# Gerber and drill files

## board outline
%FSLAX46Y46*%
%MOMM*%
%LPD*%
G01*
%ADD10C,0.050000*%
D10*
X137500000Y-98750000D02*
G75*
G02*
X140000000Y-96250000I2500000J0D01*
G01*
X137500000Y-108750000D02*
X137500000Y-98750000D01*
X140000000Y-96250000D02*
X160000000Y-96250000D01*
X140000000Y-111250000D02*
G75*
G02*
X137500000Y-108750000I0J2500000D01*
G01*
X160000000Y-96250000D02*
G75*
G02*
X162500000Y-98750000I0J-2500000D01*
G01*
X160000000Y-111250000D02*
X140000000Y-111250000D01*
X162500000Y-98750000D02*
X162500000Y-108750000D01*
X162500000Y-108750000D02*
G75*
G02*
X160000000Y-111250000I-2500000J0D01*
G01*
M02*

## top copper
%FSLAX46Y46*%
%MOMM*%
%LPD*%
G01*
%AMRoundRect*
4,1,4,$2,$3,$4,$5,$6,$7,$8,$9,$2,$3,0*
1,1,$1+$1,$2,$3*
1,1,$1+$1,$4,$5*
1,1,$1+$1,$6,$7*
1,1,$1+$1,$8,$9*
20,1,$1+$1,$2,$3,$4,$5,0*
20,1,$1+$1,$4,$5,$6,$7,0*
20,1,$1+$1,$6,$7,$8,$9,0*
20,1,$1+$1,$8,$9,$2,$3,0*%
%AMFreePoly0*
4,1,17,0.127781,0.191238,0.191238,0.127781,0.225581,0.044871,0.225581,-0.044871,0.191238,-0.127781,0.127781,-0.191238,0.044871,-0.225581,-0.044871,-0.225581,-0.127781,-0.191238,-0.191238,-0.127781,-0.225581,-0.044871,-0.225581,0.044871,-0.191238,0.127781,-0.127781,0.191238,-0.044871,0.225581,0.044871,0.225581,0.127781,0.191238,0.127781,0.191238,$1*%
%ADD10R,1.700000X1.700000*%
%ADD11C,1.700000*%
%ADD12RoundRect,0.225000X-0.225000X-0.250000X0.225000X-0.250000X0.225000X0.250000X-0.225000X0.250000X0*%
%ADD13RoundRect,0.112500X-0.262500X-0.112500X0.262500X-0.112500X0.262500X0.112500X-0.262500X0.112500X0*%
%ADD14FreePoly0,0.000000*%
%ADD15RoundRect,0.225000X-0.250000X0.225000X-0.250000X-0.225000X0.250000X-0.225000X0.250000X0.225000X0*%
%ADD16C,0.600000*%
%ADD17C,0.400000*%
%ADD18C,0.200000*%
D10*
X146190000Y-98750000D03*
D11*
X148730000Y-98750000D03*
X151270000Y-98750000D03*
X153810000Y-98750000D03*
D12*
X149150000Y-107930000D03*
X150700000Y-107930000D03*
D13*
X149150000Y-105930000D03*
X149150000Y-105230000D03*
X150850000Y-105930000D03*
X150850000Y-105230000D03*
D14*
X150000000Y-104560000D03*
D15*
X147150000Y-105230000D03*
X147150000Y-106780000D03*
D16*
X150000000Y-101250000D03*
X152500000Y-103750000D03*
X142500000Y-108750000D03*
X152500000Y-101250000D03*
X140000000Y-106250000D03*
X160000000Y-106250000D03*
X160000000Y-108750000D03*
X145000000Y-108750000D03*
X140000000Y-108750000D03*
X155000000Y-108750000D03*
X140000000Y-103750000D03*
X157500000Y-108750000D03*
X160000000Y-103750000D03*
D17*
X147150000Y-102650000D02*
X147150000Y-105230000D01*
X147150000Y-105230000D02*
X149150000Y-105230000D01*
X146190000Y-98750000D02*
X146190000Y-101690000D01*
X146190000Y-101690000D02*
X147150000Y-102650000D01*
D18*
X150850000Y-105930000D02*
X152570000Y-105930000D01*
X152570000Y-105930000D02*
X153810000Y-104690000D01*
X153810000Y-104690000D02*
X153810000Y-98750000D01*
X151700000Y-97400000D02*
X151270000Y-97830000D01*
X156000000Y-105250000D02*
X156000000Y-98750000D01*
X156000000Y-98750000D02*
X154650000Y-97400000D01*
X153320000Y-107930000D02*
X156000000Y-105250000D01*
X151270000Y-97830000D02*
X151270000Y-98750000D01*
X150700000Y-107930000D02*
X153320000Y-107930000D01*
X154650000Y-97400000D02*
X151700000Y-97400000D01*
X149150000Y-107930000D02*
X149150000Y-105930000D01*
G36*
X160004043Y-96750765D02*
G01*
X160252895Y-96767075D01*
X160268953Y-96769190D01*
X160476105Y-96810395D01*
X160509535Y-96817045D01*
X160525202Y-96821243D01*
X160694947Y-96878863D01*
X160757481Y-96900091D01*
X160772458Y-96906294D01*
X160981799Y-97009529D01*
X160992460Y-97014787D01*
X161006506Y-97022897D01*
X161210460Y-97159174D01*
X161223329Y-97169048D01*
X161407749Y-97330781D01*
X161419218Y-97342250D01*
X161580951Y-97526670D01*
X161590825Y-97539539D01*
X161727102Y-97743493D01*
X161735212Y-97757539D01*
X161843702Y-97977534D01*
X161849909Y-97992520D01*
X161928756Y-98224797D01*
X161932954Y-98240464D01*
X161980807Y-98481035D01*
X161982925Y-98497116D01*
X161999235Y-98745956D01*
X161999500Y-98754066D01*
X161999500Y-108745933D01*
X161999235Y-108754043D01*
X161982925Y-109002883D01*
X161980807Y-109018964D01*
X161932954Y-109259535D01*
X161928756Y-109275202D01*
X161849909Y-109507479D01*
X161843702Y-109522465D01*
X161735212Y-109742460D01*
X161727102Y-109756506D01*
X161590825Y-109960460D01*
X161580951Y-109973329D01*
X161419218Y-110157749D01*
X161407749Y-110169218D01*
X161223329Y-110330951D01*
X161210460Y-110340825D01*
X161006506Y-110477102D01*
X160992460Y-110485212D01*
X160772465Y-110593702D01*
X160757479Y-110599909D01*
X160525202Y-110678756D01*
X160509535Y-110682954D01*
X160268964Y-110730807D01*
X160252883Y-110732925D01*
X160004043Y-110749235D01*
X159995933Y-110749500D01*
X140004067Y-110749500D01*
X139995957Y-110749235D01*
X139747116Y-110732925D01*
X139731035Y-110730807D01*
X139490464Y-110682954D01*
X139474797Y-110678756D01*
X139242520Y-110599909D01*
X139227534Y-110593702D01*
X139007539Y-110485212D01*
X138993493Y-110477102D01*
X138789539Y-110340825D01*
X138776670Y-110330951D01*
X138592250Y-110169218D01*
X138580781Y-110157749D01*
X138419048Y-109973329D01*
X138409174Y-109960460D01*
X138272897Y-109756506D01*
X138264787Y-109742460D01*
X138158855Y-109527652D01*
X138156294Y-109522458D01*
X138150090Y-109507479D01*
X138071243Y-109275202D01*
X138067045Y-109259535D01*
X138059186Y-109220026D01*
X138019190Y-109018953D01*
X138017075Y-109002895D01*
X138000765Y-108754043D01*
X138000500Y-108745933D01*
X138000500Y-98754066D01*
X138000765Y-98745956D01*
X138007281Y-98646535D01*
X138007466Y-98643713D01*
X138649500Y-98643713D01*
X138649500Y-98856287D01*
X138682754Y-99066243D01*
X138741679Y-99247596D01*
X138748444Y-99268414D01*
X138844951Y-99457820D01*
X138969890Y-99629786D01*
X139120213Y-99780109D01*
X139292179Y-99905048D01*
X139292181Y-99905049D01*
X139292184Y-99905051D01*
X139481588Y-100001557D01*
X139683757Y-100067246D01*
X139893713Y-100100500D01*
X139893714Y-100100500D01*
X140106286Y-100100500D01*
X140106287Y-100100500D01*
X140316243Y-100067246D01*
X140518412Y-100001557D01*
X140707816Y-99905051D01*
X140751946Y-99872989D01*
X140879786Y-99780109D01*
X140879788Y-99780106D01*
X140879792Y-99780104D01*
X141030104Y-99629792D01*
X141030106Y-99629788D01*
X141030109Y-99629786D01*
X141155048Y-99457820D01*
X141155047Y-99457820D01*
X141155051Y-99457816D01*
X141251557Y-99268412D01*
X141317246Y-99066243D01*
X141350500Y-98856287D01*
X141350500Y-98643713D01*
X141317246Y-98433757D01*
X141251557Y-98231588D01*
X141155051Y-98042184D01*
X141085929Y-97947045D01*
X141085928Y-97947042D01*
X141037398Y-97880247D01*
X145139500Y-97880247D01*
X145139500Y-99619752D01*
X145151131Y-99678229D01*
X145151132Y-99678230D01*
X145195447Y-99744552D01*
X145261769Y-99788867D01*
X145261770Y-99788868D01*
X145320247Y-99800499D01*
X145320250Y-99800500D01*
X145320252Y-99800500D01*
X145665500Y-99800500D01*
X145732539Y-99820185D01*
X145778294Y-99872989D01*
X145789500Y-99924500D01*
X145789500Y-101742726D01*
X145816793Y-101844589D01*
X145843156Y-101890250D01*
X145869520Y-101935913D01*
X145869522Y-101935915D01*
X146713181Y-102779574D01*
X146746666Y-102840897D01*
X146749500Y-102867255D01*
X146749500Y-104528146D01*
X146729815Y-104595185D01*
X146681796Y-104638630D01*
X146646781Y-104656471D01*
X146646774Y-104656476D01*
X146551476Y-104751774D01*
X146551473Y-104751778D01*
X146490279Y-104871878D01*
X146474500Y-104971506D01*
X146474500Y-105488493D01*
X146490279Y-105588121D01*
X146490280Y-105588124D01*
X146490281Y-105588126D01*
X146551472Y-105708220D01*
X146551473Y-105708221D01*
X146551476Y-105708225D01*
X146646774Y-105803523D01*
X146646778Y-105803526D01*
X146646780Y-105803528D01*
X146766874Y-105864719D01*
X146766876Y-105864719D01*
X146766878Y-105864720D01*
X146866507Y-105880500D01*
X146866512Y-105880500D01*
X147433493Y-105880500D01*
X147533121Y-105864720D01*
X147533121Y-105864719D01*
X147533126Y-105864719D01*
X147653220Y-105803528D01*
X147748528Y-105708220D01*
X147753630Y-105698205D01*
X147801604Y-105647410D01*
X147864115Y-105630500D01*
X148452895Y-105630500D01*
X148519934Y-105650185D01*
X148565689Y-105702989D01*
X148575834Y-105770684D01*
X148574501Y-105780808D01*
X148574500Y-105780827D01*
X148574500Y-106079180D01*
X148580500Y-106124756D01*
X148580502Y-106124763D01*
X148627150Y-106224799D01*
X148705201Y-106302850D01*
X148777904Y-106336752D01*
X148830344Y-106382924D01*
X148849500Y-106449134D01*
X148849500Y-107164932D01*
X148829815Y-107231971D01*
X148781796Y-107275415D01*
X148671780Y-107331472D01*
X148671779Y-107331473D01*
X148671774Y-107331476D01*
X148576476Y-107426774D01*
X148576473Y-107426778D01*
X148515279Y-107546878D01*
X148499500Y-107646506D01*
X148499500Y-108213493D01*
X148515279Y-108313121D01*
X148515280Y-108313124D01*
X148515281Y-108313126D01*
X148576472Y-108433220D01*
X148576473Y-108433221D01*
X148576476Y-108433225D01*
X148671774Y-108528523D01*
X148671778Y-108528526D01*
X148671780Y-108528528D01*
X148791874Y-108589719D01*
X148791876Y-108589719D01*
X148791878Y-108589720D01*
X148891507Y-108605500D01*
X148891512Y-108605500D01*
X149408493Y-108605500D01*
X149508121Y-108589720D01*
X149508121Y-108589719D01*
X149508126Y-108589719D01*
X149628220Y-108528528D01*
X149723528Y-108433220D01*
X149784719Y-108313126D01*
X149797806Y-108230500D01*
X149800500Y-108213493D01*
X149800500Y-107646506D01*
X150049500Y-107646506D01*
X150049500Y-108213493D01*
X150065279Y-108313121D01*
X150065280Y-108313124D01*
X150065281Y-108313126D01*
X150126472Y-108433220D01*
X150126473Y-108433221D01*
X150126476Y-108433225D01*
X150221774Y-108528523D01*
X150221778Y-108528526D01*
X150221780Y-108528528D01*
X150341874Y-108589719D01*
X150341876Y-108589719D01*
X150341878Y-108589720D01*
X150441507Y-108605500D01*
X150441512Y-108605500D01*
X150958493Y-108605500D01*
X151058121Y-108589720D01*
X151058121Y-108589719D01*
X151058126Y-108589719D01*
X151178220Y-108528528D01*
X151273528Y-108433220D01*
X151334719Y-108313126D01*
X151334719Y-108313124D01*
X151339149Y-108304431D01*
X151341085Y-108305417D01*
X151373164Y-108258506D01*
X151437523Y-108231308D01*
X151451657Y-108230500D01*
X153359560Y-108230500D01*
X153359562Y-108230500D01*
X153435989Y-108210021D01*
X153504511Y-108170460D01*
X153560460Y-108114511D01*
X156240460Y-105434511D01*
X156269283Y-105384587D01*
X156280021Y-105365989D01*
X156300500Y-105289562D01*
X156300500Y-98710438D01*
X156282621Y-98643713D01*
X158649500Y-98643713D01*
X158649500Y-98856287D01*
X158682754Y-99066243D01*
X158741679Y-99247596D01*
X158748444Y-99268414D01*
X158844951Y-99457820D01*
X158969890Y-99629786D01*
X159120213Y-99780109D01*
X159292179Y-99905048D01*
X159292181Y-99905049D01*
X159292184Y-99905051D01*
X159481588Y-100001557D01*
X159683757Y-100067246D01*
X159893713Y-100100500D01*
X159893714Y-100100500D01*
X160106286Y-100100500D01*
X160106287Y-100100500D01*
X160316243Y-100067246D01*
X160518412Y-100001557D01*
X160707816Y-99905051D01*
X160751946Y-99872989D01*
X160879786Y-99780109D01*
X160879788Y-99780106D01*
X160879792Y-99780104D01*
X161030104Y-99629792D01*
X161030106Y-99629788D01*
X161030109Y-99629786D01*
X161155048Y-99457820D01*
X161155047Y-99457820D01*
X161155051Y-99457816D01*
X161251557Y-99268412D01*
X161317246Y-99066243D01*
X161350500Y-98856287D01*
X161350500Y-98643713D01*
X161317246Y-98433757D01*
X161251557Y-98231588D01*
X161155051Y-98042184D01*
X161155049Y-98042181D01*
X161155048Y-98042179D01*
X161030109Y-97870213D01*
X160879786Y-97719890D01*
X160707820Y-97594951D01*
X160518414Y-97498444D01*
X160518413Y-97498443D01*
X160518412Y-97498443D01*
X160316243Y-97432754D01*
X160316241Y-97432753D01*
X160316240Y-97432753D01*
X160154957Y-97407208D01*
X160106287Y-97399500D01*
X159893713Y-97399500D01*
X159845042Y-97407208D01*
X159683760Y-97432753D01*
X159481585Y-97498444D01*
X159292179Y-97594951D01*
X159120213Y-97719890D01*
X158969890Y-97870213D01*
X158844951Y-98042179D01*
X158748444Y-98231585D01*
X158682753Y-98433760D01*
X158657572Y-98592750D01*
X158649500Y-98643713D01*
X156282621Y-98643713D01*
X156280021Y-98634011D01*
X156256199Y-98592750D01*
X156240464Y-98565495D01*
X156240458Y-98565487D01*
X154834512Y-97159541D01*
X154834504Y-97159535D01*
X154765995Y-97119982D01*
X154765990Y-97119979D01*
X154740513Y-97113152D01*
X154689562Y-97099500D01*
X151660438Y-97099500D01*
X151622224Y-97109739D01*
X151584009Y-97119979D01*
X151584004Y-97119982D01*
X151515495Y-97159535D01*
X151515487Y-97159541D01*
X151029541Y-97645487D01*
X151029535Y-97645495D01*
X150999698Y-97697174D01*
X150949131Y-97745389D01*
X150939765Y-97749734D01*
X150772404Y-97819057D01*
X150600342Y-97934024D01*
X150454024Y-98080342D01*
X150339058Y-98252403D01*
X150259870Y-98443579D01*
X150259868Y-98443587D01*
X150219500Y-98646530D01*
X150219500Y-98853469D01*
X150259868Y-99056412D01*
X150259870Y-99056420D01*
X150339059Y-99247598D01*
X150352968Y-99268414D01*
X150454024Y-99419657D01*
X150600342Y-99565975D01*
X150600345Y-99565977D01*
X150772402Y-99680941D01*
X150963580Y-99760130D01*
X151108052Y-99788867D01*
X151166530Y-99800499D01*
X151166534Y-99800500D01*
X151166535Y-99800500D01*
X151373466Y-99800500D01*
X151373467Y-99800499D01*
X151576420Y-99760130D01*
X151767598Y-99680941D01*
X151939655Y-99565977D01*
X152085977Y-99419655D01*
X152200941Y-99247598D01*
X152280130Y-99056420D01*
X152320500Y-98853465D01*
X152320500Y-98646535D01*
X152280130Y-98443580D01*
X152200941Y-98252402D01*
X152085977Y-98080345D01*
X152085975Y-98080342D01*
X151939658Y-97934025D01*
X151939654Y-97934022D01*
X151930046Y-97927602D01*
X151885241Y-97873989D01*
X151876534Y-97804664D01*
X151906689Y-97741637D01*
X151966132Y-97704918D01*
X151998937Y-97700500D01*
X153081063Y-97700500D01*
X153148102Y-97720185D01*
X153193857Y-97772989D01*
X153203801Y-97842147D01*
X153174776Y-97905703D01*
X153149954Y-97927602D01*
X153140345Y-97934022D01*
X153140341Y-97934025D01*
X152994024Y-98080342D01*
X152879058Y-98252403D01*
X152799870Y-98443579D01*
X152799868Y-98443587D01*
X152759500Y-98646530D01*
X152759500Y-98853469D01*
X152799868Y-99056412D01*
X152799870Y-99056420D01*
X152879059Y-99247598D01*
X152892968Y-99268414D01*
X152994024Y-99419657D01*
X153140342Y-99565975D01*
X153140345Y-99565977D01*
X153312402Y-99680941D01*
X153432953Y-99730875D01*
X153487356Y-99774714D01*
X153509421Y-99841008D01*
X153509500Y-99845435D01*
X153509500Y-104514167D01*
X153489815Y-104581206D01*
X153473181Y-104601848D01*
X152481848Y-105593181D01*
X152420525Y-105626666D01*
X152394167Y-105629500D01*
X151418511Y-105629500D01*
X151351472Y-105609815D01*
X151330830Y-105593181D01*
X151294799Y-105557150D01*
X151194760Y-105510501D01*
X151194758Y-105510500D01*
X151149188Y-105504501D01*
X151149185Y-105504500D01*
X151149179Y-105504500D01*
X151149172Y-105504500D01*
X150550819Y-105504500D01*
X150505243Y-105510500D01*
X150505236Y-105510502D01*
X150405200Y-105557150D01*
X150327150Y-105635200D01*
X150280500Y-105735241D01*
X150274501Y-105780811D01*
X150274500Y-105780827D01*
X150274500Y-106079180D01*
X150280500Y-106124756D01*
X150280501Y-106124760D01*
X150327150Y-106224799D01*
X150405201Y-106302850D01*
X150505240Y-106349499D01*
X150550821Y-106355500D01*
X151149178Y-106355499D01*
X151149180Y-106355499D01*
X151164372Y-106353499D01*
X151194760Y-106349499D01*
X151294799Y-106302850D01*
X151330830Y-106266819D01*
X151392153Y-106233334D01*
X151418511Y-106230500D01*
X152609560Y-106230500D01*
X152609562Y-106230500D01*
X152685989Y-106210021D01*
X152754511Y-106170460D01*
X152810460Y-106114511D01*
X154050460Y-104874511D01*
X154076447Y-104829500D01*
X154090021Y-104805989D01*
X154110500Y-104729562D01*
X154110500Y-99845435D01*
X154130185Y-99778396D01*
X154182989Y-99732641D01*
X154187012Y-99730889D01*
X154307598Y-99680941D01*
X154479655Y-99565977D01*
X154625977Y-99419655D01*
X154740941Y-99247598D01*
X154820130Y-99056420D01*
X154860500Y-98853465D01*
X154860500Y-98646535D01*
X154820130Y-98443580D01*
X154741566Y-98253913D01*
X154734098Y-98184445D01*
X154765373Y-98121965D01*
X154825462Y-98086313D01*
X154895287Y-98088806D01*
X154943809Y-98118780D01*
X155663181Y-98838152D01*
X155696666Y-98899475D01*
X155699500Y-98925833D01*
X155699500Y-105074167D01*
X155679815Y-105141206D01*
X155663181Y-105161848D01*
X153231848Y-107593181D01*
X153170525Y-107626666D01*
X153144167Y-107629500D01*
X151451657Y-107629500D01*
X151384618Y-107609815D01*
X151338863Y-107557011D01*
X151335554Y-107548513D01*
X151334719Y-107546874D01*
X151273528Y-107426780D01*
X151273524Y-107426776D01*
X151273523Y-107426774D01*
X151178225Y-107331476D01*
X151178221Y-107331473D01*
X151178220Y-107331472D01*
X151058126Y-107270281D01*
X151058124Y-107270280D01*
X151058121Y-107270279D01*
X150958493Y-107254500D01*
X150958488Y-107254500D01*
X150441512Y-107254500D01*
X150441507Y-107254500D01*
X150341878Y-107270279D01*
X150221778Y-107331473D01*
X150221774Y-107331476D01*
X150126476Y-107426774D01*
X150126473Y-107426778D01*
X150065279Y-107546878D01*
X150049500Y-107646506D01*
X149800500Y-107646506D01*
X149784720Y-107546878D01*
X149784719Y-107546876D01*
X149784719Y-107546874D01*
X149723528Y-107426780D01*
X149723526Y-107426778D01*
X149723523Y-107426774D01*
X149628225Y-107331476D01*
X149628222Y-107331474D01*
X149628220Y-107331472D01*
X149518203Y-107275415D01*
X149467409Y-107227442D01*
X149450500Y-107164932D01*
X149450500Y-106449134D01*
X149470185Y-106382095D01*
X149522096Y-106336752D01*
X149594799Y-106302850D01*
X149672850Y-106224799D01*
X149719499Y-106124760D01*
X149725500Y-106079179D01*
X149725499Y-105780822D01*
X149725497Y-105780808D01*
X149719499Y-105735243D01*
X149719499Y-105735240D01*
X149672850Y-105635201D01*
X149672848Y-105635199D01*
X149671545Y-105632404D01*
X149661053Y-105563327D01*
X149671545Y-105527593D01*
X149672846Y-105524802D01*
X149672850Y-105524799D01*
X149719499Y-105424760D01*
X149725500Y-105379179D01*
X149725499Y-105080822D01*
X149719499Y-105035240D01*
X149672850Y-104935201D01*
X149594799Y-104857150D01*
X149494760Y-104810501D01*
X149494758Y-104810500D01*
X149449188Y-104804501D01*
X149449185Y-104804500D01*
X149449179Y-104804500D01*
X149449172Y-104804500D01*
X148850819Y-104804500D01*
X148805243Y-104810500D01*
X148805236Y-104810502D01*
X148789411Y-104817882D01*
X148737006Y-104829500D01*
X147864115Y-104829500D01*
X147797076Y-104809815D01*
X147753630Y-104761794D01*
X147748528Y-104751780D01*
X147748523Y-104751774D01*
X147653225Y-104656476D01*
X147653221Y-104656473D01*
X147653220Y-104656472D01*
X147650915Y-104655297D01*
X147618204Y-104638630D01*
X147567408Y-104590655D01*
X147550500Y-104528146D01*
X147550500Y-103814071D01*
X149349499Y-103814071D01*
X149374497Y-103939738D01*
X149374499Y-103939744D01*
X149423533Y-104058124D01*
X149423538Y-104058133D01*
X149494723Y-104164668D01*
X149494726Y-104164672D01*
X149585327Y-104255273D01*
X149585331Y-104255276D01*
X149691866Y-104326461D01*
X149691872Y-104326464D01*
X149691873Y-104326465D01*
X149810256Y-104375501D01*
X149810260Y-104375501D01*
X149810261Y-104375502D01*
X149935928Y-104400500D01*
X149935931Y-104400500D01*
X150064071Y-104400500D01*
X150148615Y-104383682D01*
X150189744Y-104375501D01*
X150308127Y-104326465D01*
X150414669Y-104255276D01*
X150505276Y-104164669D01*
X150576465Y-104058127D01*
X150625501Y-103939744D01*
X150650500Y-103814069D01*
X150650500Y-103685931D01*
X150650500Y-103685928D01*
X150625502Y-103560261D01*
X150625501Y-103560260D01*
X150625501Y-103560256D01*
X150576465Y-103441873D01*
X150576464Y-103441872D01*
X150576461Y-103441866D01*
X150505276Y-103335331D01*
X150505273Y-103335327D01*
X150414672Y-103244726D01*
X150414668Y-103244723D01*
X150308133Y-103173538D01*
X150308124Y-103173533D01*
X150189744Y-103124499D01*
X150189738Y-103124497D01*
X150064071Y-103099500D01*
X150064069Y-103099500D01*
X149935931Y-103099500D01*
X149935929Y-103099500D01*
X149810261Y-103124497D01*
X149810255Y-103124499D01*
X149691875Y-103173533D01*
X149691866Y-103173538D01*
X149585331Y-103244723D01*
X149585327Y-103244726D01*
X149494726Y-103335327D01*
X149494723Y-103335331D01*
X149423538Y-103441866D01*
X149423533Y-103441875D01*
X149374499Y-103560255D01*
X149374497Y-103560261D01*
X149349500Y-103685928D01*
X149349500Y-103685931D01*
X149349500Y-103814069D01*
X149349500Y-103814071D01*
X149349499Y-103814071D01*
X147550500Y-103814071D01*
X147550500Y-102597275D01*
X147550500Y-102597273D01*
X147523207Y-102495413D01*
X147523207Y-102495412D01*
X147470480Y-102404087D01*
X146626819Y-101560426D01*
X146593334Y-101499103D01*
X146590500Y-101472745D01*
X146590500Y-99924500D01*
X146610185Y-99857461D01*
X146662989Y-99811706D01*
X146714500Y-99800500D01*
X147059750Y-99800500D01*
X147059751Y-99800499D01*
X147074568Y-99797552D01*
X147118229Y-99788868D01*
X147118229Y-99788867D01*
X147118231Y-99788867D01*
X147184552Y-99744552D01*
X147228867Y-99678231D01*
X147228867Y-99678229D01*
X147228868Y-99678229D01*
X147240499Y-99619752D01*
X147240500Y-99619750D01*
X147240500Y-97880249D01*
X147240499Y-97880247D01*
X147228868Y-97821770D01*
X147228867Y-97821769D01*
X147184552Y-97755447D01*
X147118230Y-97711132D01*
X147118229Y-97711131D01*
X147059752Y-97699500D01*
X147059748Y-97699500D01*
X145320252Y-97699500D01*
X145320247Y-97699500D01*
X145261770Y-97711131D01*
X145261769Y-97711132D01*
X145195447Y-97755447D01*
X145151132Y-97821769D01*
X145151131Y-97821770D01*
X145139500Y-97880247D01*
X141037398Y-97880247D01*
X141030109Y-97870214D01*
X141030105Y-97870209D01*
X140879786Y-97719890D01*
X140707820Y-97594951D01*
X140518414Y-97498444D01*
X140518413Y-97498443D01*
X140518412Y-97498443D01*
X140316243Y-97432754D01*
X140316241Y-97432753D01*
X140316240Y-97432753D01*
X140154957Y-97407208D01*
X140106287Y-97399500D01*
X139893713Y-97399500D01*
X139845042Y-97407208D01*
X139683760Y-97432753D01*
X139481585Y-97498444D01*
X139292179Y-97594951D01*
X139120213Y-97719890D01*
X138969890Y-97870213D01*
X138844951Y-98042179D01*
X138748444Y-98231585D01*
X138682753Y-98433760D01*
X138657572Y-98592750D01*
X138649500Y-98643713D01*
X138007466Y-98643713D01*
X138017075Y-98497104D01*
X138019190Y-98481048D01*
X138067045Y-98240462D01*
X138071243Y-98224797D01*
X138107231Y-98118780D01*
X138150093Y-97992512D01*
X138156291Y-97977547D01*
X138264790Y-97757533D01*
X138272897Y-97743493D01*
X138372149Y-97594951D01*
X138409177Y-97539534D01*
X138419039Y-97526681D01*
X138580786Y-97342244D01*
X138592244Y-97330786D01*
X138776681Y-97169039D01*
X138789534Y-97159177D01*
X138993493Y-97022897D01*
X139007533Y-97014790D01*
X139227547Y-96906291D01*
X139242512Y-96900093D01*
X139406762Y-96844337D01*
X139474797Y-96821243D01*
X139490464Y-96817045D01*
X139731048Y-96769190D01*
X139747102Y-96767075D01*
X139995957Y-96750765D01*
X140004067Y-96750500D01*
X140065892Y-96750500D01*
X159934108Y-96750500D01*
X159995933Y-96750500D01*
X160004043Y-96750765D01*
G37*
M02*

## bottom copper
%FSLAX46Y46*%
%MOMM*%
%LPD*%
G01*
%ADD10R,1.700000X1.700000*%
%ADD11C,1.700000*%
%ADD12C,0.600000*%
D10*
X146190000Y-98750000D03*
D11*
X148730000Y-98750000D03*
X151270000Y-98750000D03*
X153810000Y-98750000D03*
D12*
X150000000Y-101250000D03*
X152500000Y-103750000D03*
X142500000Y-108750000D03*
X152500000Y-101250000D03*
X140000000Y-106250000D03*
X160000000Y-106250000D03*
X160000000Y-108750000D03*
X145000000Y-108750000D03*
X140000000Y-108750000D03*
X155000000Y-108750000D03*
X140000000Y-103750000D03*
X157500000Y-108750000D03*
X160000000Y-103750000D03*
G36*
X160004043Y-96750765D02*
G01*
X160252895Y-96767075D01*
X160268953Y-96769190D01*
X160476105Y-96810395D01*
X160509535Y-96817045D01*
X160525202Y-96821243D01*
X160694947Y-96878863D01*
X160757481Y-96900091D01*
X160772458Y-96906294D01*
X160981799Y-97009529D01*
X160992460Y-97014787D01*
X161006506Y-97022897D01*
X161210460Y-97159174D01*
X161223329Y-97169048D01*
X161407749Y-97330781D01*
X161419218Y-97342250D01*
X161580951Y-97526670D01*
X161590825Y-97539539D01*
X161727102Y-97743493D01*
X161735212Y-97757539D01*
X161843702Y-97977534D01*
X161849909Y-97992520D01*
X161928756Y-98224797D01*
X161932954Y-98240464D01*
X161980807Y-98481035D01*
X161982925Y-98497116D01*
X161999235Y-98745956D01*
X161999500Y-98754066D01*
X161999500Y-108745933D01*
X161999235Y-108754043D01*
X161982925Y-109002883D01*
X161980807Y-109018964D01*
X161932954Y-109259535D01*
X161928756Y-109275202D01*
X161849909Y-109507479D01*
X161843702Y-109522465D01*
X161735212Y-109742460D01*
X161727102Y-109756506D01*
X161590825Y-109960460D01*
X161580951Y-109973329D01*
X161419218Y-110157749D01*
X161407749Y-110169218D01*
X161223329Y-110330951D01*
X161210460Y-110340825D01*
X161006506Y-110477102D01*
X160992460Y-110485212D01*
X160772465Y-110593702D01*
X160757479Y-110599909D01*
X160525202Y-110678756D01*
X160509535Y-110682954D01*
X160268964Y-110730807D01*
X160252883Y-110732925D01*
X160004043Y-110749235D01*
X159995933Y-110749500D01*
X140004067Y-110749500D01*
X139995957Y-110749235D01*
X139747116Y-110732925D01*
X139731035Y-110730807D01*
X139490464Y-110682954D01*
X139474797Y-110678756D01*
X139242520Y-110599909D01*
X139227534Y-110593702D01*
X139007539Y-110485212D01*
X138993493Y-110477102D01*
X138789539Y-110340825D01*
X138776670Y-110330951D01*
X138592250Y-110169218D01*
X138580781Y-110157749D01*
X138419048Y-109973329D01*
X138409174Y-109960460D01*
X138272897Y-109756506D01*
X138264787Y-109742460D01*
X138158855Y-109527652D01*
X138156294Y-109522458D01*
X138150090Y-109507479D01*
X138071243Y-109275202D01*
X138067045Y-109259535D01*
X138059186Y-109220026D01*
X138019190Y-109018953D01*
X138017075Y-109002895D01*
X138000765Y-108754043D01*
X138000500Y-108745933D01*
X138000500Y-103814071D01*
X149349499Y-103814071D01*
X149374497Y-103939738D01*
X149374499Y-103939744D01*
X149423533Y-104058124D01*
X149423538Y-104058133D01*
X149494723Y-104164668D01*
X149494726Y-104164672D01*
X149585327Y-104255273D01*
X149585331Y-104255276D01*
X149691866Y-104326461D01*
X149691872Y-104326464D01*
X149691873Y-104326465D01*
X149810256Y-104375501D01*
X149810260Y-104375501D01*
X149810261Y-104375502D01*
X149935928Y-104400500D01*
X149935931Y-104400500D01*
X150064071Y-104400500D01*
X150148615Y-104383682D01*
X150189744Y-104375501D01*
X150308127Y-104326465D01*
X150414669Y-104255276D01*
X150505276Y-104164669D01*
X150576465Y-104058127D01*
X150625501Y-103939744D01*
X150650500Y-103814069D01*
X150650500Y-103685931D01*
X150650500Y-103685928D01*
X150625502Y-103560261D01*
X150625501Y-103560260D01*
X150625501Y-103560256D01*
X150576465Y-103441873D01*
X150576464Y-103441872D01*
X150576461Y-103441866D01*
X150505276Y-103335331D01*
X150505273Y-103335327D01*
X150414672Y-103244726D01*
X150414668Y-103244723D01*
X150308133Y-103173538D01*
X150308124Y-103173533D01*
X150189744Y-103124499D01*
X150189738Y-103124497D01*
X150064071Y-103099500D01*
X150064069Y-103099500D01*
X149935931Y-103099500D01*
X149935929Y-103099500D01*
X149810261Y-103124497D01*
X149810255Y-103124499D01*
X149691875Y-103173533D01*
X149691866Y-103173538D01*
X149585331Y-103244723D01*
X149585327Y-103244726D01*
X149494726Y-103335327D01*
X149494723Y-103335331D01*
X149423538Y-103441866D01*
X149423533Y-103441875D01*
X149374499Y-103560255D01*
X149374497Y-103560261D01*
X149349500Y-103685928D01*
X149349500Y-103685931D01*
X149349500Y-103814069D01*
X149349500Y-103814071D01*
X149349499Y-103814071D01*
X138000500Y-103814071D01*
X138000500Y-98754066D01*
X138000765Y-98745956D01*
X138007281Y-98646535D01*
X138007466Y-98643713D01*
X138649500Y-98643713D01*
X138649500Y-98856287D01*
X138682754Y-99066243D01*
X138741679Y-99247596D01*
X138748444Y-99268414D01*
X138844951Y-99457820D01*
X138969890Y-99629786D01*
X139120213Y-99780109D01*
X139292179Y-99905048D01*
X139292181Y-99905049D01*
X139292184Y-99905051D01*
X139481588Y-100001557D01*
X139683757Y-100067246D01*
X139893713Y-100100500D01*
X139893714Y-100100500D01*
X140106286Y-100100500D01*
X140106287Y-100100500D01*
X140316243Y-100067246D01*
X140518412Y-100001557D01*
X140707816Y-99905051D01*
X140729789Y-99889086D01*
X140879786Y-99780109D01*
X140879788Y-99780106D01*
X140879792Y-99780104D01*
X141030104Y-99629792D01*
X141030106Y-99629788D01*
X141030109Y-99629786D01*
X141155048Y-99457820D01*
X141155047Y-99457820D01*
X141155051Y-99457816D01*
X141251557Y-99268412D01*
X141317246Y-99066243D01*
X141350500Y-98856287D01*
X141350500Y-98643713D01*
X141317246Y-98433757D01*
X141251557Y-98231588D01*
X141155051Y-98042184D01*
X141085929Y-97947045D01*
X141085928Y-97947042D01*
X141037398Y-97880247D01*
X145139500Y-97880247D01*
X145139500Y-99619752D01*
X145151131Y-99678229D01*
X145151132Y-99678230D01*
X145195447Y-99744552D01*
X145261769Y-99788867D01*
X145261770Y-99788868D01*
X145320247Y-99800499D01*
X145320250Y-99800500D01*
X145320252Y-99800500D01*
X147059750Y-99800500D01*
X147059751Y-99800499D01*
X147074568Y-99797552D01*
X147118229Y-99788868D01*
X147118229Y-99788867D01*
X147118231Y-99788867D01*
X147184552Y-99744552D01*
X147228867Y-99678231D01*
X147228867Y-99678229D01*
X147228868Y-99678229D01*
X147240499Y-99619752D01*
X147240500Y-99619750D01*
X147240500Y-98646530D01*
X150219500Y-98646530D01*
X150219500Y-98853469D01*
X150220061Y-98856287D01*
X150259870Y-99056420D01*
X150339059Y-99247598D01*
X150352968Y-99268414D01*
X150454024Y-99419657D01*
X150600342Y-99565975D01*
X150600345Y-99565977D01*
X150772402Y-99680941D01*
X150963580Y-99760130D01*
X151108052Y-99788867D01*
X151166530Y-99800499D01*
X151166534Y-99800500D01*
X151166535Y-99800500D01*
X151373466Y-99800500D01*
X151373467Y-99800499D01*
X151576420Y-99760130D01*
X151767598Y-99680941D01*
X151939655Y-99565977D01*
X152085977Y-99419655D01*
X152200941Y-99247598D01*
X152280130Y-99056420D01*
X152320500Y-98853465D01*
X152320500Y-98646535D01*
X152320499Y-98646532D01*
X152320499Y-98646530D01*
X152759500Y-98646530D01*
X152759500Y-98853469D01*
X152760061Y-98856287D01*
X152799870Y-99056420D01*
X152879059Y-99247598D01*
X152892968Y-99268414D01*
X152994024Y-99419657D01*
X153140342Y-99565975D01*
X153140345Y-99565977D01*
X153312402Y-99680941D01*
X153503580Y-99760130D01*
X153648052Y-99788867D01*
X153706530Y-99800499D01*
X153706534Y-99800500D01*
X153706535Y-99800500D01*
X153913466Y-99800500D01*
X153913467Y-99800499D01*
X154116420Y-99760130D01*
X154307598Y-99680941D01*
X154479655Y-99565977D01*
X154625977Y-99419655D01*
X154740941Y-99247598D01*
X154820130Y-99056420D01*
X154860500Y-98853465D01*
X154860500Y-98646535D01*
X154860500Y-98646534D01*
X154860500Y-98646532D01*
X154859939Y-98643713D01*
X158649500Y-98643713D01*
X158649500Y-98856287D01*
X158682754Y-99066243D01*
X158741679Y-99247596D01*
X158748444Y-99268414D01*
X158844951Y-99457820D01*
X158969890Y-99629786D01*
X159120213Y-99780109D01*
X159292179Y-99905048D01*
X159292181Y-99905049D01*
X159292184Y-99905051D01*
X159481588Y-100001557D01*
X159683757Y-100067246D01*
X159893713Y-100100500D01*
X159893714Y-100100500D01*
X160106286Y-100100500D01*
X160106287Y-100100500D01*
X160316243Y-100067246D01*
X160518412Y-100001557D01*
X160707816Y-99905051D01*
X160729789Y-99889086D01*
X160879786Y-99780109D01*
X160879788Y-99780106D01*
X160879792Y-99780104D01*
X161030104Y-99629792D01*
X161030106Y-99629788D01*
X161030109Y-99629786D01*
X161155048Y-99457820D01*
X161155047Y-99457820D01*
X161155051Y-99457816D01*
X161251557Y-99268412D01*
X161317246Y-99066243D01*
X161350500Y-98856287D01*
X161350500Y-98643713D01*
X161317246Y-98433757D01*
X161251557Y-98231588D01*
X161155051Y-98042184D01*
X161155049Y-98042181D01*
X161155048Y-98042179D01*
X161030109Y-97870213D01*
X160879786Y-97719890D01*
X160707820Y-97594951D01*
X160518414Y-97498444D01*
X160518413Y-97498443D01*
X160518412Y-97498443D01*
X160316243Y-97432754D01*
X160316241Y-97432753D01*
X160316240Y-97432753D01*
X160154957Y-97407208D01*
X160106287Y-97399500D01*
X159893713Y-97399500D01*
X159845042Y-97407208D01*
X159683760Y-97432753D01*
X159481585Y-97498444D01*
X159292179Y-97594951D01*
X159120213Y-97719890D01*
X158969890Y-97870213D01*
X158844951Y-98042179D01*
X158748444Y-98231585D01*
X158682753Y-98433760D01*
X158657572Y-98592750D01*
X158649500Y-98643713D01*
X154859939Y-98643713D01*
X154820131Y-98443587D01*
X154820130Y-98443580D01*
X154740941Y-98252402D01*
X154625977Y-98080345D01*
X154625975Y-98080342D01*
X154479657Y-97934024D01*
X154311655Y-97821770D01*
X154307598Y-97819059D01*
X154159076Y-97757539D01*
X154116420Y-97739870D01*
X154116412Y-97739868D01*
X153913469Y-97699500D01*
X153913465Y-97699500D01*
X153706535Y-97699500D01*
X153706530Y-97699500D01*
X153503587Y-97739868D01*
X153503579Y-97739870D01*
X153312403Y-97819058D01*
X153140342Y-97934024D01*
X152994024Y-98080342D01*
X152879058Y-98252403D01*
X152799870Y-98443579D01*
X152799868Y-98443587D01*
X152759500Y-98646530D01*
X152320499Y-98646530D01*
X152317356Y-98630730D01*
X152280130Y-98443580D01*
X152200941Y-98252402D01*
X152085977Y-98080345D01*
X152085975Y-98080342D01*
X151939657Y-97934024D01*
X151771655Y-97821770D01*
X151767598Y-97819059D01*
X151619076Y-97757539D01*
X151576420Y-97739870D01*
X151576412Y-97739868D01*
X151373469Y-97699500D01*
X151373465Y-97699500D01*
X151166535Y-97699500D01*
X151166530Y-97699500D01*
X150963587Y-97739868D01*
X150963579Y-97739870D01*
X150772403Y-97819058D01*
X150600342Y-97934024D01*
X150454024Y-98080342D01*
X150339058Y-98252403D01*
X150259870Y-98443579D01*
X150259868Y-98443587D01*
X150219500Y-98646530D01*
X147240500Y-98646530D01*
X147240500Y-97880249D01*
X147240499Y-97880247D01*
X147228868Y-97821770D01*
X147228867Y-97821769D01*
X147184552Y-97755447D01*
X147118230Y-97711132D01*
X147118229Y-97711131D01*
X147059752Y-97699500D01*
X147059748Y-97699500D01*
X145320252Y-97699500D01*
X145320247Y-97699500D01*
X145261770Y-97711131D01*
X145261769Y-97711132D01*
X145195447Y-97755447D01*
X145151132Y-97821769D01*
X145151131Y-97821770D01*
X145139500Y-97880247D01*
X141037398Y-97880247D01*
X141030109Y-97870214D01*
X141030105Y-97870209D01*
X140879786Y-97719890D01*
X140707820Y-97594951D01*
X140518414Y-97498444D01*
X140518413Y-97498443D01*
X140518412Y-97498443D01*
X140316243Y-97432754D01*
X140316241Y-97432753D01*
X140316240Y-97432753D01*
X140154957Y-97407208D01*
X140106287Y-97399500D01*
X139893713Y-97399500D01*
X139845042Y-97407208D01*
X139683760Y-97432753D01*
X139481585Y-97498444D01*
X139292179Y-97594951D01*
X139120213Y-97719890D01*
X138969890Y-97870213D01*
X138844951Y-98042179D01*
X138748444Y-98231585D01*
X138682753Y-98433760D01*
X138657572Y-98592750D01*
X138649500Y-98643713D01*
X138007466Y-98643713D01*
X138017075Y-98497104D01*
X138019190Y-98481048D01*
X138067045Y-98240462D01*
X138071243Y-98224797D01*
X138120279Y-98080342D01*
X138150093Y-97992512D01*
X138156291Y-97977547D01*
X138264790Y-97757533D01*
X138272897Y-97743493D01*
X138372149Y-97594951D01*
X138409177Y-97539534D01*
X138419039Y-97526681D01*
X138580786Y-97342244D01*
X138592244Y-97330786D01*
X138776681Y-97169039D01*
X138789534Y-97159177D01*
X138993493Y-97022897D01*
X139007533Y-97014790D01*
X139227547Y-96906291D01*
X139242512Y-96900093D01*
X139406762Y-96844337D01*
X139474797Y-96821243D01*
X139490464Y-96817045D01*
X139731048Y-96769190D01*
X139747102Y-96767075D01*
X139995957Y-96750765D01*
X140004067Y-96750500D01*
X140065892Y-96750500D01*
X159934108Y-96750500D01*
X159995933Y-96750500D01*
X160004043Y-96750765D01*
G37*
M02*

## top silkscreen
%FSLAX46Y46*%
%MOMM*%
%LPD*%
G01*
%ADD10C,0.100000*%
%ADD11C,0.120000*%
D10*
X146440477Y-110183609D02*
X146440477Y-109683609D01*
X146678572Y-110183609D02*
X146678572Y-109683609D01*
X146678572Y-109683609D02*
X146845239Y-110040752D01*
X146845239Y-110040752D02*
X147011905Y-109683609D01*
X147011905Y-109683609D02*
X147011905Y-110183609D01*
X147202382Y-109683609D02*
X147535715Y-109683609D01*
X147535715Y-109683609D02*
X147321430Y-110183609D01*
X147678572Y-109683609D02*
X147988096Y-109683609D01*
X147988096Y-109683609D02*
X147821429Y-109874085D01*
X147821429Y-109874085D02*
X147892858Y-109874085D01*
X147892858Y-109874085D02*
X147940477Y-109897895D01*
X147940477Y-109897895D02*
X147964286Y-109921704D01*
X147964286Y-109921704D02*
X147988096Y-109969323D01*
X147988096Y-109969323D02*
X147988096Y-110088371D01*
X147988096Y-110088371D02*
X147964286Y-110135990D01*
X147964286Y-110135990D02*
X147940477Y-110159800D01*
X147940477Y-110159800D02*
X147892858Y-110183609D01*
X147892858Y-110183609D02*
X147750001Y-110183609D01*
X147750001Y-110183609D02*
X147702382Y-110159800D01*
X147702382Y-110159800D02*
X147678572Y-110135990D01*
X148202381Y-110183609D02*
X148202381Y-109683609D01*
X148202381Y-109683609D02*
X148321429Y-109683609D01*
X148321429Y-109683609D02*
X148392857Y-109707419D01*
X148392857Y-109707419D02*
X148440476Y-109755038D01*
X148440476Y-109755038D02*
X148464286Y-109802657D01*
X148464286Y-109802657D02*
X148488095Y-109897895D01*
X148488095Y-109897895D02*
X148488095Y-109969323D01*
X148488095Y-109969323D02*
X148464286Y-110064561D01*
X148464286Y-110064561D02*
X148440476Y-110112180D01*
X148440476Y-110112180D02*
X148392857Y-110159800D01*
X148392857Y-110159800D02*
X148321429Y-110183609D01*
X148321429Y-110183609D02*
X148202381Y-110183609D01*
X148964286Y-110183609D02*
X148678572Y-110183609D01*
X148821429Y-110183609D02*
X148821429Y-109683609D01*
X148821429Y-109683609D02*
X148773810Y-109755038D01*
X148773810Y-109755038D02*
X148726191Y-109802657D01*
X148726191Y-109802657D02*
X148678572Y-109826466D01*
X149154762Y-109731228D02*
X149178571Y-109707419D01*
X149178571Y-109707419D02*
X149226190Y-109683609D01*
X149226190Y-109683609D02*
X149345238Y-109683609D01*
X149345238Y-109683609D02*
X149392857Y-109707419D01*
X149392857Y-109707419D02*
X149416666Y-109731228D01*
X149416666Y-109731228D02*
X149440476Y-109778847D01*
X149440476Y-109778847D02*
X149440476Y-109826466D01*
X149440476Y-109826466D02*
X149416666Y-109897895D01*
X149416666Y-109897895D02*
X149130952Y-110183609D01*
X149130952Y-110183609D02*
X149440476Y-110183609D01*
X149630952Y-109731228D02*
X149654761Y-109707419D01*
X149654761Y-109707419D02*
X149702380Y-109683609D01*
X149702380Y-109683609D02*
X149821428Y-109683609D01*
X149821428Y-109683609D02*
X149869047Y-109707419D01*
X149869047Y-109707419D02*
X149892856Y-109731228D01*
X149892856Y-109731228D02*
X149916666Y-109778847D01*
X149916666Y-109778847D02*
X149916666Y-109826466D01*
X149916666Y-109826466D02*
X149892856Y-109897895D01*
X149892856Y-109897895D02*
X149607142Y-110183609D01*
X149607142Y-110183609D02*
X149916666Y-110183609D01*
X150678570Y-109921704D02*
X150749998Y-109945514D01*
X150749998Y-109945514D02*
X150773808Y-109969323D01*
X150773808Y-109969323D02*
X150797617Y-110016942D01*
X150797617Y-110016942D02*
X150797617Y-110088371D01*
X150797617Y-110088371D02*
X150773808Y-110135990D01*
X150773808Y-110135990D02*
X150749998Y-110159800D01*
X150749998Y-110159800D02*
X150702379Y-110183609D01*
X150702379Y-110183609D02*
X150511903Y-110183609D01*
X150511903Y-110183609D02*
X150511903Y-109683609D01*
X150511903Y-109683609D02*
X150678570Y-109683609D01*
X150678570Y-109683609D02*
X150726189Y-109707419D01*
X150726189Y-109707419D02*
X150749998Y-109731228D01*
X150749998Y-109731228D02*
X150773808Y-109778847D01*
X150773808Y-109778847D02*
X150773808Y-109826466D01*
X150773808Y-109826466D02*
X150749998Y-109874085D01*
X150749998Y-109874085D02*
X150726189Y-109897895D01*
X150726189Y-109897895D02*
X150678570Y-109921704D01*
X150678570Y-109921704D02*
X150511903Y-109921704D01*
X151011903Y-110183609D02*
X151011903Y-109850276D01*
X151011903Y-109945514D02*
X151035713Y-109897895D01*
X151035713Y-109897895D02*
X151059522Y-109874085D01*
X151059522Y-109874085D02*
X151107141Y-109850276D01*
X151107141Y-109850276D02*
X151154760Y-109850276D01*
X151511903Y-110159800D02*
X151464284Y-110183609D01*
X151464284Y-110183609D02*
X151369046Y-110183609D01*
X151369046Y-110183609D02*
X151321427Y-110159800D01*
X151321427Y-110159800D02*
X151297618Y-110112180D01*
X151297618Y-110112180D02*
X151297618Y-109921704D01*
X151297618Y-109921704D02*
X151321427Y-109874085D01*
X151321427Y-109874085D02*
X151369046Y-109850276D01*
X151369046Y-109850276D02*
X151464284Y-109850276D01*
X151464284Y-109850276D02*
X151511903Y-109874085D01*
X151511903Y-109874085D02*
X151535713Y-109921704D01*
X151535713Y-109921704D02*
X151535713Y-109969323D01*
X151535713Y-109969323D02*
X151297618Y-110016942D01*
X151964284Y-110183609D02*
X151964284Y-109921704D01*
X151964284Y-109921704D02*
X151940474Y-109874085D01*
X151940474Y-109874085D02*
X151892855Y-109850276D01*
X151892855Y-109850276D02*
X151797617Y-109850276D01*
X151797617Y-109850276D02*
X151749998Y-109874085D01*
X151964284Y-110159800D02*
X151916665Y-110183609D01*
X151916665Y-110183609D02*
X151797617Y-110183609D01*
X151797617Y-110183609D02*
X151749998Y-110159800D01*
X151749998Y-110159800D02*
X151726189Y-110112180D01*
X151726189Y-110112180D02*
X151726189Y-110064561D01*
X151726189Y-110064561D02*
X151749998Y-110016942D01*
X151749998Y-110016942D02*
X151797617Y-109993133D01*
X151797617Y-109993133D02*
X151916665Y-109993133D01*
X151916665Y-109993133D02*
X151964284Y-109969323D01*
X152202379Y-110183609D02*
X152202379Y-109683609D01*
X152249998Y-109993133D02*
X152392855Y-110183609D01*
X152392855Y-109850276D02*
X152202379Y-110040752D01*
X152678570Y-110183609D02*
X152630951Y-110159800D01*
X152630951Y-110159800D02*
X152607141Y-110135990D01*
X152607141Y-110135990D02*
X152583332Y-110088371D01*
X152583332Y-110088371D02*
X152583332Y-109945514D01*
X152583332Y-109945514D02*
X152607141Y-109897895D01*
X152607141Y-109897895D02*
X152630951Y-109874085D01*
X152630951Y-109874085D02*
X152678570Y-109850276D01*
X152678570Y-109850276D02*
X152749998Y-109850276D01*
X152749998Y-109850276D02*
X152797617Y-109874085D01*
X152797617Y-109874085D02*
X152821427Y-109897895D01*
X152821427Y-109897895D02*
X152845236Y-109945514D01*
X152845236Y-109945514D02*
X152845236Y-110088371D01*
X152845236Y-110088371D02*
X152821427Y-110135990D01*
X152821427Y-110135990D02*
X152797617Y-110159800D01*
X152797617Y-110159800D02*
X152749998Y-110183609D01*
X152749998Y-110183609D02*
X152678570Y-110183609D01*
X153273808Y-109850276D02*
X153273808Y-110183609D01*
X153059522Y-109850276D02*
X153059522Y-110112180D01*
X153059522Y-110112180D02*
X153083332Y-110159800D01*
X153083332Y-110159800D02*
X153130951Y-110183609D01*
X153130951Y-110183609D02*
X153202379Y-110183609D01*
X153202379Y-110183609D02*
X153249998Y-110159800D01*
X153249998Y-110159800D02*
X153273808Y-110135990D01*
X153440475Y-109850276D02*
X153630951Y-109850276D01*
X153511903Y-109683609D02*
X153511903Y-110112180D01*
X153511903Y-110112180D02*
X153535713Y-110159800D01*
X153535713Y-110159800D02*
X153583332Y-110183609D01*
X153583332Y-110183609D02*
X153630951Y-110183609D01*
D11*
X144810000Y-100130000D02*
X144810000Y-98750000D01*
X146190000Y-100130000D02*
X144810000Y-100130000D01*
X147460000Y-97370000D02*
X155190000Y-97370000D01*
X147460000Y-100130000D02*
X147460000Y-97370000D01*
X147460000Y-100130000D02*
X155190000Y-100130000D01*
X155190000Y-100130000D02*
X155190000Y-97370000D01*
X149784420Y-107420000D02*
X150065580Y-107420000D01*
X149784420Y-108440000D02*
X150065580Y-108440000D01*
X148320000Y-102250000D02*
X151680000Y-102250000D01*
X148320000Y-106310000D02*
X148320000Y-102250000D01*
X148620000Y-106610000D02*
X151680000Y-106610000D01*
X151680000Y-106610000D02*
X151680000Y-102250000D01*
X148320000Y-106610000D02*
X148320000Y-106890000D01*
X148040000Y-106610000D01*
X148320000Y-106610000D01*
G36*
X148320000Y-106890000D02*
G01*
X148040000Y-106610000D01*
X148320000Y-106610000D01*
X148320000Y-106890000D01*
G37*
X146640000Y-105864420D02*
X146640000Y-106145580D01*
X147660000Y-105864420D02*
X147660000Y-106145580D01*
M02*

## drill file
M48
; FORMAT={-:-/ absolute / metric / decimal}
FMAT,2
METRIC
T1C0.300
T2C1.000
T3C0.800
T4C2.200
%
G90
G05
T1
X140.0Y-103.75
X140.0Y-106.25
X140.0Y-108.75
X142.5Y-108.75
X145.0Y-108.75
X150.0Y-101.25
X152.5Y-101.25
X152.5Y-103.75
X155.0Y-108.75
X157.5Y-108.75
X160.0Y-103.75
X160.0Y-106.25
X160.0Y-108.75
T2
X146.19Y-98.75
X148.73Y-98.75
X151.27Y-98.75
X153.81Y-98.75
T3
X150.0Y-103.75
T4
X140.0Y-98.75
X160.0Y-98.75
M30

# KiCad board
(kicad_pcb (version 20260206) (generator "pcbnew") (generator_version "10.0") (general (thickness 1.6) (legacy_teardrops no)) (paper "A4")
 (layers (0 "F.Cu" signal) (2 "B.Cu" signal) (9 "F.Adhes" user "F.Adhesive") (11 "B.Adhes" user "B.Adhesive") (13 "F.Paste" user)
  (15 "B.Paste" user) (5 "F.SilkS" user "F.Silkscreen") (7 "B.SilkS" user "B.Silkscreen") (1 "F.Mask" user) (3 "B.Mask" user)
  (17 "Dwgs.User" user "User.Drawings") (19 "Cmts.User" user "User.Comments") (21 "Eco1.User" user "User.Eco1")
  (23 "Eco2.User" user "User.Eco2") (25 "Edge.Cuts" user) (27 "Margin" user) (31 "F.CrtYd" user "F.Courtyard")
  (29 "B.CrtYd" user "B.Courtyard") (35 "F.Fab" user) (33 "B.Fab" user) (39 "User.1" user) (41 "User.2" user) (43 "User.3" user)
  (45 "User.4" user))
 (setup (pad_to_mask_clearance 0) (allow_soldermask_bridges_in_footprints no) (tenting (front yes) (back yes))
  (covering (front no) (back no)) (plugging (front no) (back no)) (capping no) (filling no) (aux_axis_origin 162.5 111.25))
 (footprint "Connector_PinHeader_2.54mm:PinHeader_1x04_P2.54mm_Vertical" (layer "F.Cu") (at 146.19 98.75 90)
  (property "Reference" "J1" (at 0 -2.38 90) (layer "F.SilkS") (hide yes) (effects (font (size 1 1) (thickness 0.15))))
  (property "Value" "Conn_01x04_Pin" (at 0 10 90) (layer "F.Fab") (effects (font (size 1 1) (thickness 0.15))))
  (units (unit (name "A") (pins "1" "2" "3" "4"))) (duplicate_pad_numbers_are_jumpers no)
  (fp_line (start -1.38 -1.38) (end 0 -1.38) (stroke (width 0.12) (type solid)) (layer "F.SilkS"))
  (fp_line (start -1.38 0) (end -1.38 -1.38) (stroke (width 0.12) (type solid)) (layer "F.SilkS"))
  (fp_line (start 1.38 1.27) (end 1.38 9) (stroke (width 0.12) (type solid)) (layer "F.SilkS"))
  (fp_line (start -1.38 1.27) (end 1.38 1.27) (stroke (width 0.12) (type solid)) (layer "F.SilkS"))
  (fp_line (start -1.38 1.27) (end -1.38 9) (stroke (width 0.12) (type solid)) (layer "F.SilkS"))
  (fp_line (start -1.38 9) (end 1.38 9) (stroke (width 0.12) (type solid)) (layer "F.SilkS"))
  (pad "1" thru_hole rect (at 0 0 90) (size 1.7 1.7) (drill 1) (layers "*.Cu" "*.Mask") (remove_unused_layers no) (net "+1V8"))
  (pad "2" thru_hole circle (at 0 2.54 90) (size 1.7 1.7) (drill 1) (layers "*.Cu" "*.Mask") (remove_unused_layers no) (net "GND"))
  (pad "3" thru_hole circle (at 0 5.08 90) (size 1.7 1.7) (drill 1) (layers "*.Cu" "*.Mask") (remove_unused_layers no) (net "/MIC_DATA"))
  (pad "4" thru_hole circle (at 0 7.62 90) (size 1.7 1.7) (drill 1) (layers "*.Cu" "*.Mask") (remove_unused_layers no) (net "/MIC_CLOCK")))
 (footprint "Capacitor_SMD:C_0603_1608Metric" (layer "F.Cu") (at 149.925 107.93)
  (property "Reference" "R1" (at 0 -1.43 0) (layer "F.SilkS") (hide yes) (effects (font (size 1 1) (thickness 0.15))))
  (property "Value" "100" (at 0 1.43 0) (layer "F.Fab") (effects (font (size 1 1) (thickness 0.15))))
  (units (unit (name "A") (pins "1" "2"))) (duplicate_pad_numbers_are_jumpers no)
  (fp_line (start -0.14058 -0.51) (end 0.14058 -0.51) (stroke (width 0.12) (type solid)) (layer "F.SilkS"))
  (fp_line (start -0.14058 0.51) (end 0.14058 0.51) (stroke (width 0.12) (type solid)) (layer "F.SilkS"))
  (pad "1" smd roundrect (at -0.775 0) (size 0.9 0.95) (layers "F.Cu" "F.Mask" "F.Paste") (roundrect_rratio 0.25) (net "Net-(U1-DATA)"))
  (pad "2" smd roundrect (at 0.775 0) (size 0.9 0.95) (layers "F.Cu" "F.Mask" "F.Paste") (roundrect_rratio 0.25) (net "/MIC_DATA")))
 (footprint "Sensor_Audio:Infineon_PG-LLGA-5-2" (layer "F.Cu") (at 150 104.43 90)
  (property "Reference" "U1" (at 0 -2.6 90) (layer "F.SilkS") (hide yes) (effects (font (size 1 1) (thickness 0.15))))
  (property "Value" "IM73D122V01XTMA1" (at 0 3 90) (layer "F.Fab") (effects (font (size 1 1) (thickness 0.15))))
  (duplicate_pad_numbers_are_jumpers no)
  (fp_line (start 2.18 -1.68) (end 2.18 1.68) (stroke (width 0.12) (type solid)) (layer "F.SilkS"))
  (fp_line (start -1.88 -1.68) (end 2.18 -1.68) (stroke (width 0.12) (type solid)) (layer "F.SilkS"))
  (fp_line (start -2.18 -1.38) (end -2.18 1.68) (stroke (width 0.12) (type solid)) (layer "F.SilkS"))
  (fp_line (start -2.18 1.68) (end 2.18 1.68) (stroke (width 0.12) (type solid)) (layer "F.SilkS"))
  (fp_poly
   (pts (xy -2.18 -1.68) (xy -2.46 -1.68) (xy -2.18 -1.96) (xy -2.18 -1.68)) (stroke (width 0.12) (type solid)) (fill yes) (layer "F.SilkS"))
  (pad "" np_thru_hole circle (at 0.68 0 180) (size 0.8 0.8) (drill 0.8) (layers "*.Cu" "*.Mask"))
  (pad "1" smd roundrect (at -1.5 -0.85) (size 0.75 0.45) (layers "F.Cu" "F.Mask") (roundrect_rratio 0.25) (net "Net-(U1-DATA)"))
  (pad "2" smd roundrect (at -0.8 -0.85) (size 0.75 0.45) (layers "F.Cu" "F.Mask") (roundrect_rratio 0.25) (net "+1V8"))
  (pad "3" smd roundrect (at -1.5 0.85) (size 0.75 0.45) (layers "F.Cu" "F.Mask") (roundrect_rratio 0.25) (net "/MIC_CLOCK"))
  (pad "4" smd roundrect (at -0.8 0.85) (size 0.75 0.45) (layers "F.Cu" "F.Mask") (roundrect_rratio 0.25) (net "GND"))
  (pad "5" smd custom (at -0.13 0) (size 0.46 0.46) (layers "F.Cu" "F.Mask") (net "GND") (options (clearance outline) (anchor circle))
   (primitives)))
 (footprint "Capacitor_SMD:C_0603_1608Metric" (layer "F.Cu") (at 147.15 106.005 -90)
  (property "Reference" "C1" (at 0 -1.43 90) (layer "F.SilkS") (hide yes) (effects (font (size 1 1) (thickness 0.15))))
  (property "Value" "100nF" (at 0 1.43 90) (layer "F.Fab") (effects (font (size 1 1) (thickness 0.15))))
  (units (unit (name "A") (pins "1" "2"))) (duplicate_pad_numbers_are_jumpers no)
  (fp_line (start -0.14058 0.51) (end 0.14058 0.51) (stroke (width 0.12) (type solid)) (layer "F.SilkS"))
  (fp_line (start -0.14058 -0.51) (end 0.14058 -0.51) (stroke (width 0.12) (type solid)) (layer "F.SilkS"))
  (pad "1" smd roundrect (at -0.775 0 270) (size 0.9 0.95) (layers "F.Cu" "F.Mask" "F.Paste") (roundrect_rratio 0.25) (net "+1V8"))
  (pad "2" smd roundrect (at 0.775 0 270) (size 0.9 0.95) (layers "F.Cu" "F.Mask" "F.Paste") (roundrect_rratio 0.25) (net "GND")))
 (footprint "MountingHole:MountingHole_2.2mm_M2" (layer "F.Cu") (at 140 98.75)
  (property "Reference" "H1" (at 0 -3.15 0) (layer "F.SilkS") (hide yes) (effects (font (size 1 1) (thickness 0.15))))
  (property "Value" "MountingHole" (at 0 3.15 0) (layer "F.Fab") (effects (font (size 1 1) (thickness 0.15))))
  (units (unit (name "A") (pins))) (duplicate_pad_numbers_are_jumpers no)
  (pad "" np_thru_hole circle (at 0 0) (size 2.2 2.2) (drill 2.2) (layers "*.Cu" "*.Mask")))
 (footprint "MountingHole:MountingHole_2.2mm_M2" (layer "F.Cu") (at 160 98.75)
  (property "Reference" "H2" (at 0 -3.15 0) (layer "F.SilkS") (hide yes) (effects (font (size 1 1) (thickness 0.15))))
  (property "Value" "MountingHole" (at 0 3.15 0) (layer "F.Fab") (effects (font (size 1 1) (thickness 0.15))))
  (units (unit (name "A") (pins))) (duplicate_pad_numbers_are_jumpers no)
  (pad "" np_thru_hole circle (at 0 0) (size 2.2 2.2) (drill 2.2) (layers "*.Cu" "*.Mask")))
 (gr_arc (start 137.5 98.75) (mid 138.232233 96.982233) (end 140 96.25) (stroke (width 0.05) (type default)) (layer "Edge.Cuts"))
 (gr_line (start 137.5 108.75) (end 137.5 98.75) (stroke (width 0.05) (type default)) (layer "Edge.Cuts"))
 (gr_line (start 140 96.25) (end 160 96.25) (stroke (width 0.05) (type default)) (layer "Edge.Cuts"))
 (gr_arc (start 140 111.25) (mid 138.232233 110.517767) (end 137.5 108.75) (stroke (width 0.05) (type default)) (layer "Edge.Cuts"))
 (gr_arc (start 160 96.25) (mid 161.767767 96.982233) (end 162.5 98.75) (stroke (width 0.05) (type default)) (layer "Edge.Cuts"))
 (gr_line (start 160 111.25) (end 140 111.25) (stroke (width 0.05) (type default)) (layer "Edge.Cuts"))
 (gr_line (start 162.5 98.75) (end 162.5 108.75) (stroke (width 0.05) (type default)) (layer "Edge.Cuts"))
 (gr_arc (start 162.5 108.75) (mid 161.767767 110.517767) (end 160 111.25) (stroke (width 0.05) (type default)) (layer "Edge.Cuts"))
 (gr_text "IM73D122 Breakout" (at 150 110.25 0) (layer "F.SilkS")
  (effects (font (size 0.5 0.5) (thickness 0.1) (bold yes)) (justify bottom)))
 (segment (start 147.15 102.65) (end 147.15 105.23) (width 0.4) (layer "F.Cu") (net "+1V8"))
 (segment (start 147.15 105.23) (end 149.15 105.23) (width 0.4) (layer "F.Cu") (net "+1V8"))
 (segment (start 146.19 98.75) (end 146.19 101.69) (width 0.4) (layer "F.Cu") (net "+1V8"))
 (segment (start 146.19 101.69) (end 147.15 102.65) (width 0.4) (layer "F.Cu") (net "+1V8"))
 (via (at 150 101.25) (size 0.6) (drill 0.3) (layers "F.Cu" "B.Cu") (free yes) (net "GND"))
 (via (at 152.5 103.75) (size 0.6) (drill 0.3) (layers "F.Cu" "B.Cu") (free yes) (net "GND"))
 (via (at 142.5 108.75) (size 0.6) (drill 0.3) (layers "F.Cu" "B.Cu") (free yes) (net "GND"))
 (via (at 152.5 101.25) (size 0.6) (drill 0.3) (layers "F.Cu" "B.Cu") (free yes) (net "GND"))
 (via (at 140 106.25) (size 0.6) (drill 0.3) (layers "F.Cu" "B.Cu") (free yes) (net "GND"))
 (via (at 160 106.25) (size 0.6) (drill 0.3) (layers "F.Cu" "B.Cu") (free yes) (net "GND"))
 (via (at 160 108.75) (size 0.6) (drill 0.3) (layers "F.Cu" "B.Cu") (free yes) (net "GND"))
 (via (at 145 108.75) (size 0.6) (drill 0.3) (layers "F.Cu" "B.Cu") (free yes) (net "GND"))
 (via (at 140 108.75) (size 0.6) (drill 0.3) (layers "F.Cu" "B.Cu") (free yes) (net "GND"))
 (via (at 155 108.75) (size 0.6) (drill 0.3) (layers "F.Cu" "B.Cu") (free yes) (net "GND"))
 (via (at 140 103.75) (size 0.6) (drill 0.3) (layers "F.Cu" "B.Cu") (free yes) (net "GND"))
 (via (at 157.5 108.75) (size 0.6) (drill 0.3) (layers "F.Cu" "B.Cu") (free yes) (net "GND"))
 (via (at 160 103.75) (size 0.6) (drill 0.3) (layers "F.Cu" "B.Cu") (free yes) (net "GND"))
 (segment (start 150.85 105.93) (end 152.57 105.93) (width 0.2) (layer "F.Cu") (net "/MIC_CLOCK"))
 (segment (start 152.57 105.93) (end 153.81 104.69) (width 0.2) (layer "F.Cu") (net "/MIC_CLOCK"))
 (segment (start 153.81 104.69) (end 153.81 98.75) (width 0.2) (layer "F.Cu") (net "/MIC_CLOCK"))
 (segment (start 151.7 97.4) (end 151.27 97.83) (width 0.2) (layer "F.Cu") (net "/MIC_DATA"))
 (segment (start 156 105.25) (end 156 98.75) (width 0.2) (layer "F.Cu") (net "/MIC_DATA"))
 (segment (start 156 98.75) (end 154.65 97.4) (width 0.2) (layer "F.Cu") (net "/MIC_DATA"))
 (segment (start 153.32 107.93) (end 156 105.25) (width 0.2) (layer "F.Cu") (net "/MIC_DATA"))
 (segment (start 151.27 97.83) (end 151.27 98.75) (width 0.2) (layer "F.Cu") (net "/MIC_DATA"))
 (segment (start 150.7 107.93) (end 153.32 107.93) (width 0.2) (layer "F.Cu") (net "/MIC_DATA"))
 (segment (start 154.65 97.4) (end 151.7 97.4) (width 0.2) (layer "F.Cu") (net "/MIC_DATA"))
 (segment (start 149.15 107.93) (end 149.15 105.93) (width 0.2) (layer "F.Cu") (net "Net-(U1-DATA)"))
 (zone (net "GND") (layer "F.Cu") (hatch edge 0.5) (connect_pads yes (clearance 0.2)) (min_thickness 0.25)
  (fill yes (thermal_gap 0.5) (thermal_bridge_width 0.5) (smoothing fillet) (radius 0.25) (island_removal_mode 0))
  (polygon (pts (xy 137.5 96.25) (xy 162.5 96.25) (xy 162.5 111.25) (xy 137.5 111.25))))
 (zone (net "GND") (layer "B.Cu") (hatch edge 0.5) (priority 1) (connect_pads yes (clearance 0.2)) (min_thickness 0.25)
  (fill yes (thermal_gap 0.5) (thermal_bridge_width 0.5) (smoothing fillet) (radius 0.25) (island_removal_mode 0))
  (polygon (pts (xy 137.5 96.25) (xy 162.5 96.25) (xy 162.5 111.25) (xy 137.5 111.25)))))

